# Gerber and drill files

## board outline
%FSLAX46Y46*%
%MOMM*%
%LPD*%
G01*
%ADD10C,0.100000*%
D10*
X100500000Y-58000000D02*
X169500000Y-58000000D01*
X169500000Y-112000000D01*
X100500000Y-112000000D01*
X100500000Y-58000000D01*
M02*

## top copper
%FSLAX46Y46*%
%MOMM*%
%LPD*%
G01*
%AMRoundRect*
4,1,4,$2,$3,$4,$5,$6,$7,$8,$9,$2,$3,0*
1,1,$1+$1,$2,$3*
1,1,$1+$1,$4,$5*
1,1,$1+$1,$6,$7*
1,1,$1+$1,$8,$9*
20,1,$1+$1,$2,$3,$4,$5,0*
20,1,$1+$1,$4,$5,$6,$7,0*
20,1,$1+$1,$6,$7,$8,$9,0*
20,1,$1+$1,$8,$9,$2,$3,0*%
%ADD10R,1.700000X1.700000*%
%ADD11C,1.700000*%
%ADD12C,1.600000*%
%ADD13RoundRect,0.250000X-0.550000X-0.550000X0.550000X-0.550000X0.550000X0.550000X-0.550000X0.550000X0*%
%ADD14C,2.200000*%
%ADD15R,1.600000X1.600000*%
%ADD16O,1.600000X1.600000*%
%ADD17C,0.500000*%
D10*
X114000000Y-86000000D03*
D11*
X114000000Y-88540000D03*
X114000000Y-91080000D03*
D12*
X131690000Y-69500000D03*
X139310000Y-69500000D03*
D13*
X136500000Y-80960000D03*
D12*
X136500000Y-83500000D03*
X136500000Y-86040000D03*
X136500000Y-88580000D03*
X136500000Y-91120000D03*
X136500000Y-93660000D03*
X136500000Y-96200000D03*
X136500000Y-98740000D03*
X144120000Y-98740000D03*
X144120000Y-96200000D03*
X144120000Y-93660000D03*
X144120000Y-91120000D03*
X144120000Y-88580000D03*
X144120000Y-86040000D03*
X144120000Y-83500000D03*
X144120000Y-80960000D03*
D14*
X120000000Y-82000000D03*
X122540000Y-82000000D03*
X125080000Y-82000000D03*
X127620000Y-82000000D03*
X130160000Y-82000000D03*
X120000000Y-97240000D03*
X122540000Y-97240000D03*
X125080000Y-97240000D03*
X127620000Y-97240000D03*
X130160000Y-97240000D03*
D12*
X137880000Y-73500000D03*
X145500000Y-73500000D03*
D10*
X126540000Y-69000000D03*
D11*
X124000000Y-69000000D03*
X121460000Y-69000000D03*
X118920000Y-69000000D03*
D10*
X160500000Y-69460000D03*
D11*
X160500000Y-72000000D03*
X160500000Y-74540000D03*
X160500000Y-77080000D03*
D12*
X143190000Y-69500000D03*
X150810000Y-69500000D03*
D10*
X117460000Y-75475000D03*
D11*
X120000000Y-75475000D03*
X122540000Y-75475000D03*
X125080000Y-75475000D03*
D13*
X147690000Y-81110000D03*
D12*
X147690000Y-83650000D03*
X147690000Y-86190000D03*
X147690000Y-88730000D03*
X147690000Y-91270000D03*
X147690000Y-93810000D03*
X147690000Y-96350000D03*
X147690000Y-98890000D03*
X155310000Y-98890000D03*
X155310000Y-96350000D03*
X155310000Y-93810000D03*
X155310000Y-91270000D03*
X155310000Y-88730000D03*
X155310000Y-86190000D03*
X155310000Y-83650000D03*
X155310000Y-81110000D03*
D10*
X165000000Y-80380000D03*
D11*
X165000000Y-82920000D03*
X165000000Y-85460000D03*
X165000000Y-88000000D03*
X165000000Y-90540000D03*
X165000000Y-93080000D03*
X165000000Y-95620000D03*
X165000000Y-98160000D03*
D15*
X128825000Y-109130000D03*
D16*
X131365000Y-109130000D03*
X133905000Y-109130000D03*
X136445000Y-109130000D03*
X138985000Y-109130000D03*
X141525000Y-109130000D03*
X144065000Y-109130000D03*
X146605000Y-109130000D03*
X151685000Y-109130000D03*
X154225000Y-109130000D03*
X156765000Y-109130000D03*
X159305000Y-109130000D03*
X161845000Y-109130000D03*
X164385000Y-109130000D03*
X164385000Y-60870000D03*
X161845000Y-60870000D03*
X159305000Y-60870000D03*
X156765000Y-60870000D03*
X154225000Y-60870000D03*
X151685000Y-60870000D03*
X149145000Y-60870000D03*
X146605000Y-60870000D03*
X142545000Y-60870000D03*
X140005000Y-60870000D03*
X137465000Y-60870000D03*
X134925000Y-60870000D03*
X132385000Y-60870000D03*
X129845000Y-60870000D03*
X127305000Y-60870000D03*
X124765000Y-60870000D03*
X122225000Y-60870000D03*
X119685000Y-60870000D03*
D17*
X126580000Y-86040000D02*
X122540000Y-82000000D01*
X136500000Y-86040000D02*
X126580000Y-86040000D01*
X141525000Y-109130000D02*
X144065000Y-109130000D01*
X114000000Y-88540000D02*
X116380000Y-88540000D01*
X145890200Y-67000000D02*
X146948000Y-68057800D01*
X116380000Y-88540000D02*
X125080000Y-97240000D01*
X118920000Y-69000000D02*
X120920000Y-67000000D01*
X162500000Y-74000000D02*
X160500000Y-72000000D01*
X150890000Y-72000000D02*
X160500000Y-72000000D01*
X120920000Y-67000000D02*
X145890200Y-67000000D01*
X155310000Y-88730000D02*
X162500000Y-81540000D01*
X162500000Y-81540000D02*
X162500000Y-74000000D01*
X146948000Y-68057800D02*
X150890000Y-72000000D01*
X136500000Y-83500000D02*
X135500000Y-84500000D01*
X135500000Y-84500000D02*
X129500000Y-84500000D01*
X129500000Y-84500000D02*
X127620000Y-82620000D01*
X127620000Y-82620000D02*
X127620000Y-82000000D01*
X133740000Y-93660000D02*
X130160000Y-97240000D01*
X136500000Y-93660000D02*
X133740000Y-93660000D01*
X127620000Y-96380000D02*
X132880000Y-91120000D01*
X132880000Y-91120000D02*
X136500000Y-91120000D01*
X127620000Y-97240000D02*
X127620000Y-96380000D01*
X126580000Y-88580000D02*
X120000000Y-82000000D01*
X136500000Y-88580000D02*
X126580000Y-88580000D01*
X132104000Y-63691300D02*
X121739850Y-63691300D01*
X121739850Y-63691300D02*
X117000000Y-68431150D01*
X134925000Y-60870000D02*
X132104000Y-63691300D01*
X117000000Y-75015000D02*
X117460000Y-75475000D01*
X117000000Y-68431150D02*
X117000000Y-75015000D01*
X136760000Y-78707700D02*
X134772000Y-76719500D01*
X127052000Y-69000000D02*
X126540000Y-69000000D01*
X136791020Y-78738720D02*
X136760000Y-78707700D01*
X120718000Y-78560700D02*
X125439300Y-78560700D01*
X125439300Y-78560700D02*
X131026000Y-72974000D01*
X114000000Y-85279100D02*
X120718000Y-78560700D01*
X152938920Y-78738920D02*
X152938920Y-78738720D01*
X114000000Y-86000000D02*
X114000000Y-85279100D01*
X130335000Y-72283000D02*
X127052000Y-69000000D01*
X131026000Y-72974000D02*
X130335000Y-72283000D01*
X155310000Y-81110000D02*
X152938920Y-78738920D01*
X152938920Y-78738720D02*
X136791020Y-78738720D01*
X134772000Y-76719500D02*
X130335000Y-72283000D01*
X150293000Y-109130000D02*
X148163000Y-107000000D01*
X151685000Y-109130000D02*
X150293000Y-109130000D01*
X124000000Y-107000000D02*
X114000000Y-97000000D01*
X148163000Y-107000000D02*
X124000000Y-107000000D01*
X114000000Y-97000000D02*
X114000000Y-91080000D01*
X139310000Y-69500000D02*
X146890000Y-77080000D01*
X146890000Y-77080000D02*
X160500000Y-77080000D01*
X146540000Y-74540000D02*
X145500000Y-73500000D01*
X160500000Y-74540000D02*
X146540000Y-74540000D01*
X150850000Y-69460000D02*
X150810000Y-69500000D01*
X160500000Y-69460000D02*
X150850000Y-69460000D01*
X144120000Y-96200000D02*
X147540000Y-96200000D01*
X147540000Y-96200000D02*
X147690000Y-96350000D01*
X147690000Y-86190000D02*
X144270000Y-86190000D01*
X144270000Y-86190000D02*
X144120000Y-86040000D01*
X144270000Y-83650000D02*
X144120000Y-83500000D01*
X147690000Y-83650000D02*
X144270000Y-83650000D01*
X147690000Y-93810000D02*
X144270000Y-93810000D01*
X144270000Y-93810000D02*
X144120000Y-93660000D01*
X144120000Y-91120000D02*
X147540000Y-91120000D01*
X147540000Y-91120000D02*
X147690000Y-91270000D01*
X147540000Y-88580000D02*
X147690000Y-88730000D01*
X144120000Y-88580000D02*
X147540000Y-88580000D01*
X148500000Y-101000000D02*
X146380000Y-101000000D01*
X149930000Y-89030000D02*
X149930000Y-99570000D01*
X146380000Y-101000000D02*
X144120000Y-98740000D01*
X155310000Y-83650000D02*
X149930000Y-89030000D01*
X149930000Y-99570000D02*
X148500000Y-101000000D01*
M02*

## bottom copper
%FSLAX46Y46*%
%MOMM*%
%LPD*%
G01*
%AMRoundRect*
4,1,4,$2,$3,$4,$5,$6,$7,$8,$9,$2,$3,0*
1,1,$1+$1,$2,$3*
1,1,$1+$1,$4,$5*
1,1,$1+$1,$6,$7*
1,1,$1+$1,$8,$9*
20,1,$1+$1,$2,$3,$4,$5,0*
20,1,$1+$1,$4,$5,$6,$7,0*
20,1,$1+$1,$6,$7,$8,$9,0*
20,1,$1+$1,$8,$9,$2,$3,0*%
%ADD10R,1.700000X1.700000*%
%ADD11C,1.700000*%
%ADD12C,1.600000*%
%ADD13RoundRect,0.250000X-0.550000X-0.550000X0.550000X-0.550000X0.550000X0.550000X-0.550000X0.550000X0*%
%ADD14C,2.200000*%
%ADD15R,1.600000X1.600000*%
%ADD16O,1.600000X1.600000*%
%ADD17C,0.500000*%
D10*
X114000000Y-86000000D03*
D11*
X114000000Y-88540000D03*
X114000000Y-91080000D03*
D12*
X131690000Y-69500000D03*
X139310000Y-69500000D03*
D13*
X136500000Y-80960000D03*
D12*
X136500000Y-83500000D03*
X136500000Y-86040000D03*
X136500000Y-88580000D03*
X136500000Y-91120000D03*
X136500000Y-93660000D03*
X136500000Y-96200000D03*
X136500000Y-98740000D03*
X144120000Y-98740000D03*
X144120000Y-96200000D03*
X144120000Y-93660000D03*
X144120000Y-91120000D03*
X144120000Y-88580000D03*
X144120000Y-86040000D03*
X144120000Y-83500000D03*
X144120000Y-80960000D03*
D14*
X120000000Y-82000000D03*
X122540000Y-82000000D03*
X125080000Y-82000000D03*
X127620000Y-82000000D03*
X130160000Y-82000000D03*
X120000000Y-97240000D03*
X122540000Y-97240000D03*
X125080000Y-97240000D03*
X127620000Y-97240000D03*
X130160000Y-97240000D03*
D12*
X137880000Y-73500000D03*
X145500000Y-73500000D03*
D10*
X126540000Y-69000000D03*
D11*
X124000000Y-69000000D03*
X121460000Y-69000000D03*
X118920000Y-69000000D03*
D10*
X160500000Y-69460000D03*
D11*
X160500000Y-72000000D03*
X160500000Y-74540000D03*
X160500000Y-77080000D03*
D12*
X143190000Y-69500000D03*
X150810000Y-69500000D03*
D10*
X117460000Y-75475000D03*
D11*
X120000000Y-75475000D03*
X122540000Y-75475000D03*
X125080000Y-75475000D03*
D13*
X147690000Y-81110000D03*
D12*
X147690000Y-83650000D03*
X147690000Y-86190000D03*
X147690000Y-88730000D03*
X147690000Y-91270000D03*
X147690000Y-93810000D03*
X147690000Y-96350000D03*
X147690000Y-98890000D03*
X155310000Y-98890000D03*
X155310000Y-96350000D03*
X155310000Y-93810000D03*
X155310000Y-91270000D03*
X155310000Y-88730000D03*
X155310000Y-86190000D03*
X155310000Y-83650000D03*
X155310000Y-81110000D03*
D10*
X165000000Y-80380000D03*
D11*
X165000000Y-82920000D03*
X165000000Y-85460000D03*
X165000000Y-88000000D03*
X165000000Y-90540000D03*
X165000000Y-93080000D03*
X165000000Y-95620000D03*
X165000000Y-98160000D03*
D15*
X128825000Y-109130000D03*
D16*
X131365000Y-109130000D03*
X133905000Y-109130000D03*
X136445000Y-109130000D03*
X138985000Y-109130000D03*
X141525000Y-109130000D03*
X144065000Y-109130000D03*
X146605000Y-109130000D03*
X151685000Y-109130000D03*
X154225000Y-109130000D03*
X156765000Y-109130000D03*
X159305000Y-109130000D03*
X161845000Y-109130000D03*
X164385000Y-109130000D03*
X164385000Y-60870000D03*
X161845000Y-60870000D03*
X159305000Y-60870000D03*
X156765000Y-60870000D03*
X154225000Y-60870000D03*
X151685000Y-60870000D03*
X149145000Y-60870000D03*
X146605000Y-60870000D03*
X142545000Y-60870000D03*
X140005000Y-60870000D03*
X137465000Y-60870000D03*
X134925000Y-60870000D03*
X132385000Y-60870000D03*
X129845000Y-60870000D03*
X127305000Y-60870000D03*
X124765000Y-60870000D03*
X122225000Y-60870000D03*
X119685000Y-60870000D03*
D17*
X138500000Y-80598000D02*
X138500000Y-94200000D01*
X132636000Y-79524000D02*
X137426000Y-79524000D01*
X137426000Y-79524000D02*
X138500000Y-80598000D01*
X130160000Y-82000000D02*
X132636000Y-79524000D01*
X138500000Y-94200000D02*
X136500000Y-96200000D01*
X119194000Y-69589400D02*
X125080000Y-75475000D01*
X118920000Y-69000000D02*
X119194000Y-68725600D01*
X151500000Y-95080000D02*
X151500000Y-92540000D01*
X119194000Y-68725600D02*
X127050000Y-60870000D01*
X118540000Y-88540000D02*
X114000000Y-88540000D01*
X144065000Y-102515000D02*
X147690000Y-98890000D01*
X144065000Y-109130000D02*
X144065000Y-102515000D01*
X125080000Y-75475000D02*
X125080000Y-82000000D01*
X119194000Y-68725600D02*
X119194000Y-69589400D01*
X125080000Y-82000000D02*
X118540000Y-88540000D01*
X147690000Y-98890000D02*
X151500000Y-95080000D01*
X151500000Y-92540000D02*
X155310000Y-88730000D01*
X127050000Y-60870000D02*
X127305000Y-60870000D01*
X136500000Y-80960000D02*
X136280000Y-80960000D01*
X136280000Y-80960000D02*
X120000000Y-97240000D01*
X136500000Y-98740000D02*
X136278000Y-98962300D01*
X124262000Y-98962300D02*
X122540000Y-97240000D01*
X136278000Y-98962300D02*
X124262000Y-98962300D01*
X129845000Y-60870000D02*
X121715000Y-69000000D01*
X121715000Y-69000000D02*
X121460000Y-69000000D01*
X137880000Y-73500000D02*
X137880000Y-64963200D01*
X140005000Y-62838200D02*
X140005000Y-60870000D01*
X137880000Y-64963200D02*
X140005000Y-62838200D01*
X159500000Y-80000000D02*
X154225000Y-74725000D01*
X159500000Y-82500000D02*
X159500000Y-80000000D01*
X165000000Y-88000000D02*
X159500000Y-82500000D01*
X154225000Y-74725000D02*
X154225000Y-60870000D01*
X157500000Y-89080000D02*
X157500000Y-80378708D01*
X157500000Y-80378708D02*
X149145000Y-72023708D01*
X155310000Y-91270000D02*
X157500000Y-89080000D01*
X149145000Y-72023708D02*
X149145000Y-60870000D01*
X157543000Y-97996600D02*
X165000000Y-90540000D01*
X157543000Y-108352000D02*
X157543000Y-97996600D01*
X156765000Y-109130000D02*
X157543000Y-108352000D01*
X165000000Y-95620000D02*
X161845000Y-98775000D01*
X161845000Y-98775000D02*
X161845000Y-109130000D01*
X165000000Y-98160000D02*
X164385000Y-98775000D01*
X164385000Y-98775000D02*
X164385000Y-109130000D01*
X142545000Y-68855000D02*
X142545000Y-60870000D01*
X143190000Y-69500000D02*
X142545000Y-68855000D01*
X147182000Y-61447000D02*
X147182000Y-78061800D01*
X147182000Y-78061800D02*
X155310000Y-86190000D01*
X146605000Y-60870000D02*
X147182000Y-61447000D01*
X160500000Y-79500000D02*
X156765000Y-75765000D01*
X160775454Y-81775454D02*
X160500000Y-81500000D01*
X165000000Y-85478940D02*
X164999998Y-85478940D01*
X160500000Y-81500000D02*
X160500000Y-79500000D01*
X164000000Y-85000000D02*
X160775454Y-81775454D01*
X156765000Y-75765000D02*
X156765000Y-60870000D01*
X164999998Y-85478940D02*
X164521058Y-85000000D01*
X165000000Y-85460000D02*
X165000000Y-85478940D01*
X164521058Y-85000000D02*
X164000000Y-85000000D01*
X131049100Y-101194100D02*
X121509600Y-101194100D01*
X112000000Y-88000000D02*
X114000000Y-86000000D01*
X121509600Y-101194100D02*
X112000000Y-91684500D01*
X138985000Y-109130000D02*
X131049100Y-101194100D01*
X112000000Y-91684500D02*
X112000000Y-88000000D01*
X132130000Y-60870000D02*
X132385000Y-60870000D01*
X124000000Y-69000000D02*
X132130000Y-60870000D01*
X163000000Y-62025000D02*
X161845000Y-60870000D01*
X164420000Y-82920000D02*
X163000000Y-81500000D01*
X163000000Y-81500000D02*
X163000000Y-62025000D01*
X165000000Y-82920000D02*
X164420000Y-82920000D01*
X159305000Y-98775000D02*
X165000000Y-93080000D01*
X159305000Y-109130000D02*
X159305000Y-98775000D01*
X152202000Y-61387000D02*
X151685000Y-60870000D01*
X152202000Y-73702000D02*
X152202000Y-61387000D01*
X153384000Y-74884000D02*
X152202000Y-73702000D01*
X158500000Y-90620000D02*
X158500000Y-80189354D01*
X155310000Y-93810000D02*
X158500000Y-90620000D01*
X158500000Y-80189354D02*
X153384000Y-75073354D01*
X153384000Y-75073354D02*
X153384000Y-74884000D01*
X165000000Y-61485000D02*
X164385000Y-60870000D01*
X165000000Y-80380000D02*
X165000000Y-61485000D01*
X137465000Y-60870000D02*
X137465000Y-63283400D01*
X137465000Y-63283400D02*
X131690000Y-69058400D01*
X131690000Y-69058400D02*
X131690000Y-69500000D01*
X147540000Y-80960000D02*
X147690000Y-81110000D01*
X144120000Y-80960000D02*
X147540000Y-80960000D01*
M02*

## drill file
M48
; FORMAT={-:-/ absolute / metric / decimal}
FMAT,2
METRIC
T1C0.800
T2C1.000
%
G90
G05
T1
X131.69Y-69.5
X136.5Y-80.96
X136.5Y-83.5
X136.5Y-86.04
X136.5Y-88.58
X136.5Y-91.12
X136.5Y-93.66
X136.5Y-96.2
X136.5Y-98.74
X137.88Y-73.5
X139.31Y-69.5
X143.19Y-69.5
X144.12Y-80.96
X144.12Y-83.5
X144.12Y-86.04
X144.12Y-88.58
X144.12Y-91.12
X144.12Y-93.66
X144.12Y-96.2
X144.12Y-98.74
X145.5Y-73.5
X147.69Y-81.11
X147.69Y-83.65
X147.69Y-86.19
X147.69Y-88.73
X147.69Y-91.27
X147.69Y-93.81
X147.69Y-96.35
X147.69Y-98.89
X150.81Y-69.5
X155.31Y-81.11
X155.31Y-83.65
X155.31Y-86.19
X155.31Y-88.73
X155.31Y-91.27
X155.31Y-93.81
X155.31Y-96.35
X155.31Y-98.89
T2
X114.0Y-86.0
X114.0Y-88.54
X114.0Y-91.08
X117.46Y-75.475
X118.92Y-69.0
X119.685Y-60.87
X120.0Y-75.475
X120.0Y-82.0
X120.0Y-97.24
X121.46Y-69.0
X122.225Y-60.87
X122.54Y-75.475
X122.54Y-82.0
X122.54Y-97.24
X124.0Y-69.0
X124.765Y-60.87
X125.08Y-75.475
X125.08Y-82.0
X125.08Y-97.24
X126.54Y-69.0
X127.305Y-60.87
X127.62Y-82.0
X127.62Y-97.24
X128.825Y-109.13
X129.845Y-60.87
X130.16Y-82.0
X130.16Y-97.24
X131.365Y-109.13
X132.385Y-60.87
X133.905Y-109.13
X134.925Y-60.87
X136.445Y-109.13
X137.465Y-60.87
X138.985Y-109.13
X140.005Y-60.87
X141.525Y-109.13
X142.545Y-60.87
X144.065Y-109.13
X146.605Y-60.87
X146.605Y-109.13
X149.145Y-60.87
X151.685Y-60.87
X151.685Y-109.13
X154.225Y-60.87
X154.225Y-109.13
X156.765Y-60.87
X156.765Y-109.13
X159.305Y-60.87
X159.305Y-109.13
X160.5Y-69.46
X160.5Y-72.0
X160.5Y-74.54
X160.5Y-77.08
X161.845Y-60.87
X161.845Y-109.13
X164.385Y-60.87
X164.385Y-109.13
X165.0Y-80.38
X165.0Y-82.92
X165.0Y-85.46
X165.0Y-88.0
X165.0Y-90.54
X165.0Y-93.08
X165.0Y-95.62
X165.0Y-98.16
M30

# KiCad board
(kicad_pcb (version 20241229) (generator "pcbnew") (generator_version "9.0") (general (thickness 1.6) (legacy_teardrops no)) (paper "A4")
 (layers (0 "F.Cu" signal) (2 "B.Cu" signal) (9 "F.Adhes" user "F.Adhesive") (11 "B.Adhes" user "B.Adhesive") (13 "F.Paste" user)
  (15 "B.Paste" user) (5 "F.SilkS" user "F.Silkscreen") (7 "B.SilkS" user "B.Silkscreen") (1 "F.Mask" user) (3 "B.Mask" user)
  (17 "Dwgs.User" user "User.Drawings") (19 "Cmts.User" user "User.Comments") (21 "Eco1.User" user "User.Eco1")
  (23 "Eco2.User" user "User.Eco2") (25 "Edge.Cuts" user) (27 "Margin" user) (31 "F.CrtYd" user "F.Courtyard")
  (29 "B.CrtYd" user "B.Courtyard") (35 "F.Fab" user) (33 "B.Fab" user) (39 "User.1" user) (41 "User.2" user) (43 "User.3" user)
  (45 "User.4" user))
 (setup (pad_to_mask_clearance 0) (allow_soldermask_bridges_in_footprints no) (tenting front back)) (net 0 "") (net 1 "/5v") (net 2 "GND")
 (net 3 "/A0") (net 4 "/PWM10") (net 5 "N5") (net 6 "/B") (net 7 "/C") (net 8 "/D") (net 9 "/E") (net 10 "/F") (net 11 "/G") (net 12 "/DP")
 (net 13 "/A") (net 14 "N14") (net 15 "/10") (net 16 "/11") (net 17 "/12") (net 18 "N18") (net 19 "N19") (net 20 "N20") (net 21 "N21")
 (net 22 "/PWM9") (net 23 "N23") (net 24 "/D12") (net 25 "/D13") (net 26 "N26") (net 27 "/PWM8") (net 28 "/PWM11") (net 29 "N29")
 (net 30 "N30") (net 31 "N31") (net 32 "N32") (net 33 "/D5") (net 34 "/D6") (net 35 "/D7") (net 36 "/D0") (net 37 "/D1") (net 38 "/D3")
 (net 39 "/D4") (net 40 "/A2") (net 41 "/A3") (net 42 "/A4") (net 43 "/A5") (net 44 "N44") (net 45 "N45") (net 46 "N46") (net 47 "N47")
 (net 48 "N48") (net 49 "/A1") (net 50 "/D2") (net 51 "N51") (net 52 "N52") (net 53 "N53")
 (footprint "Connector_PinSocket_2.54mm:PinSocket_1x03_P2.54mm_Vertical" (layer "F.Cu") (at 114 86)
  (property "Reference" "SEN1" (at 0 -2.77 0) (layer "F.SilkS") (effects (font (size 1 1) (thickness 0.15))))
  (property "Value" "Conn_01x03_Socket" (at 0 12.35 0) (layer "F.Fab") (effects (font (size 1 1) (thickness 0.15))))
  (pad "1" thru_hole rect (at 0 0) (size 1.7 1.7) (drill 1) (layers "*.Cu" "*.Mask") (remove_unused_layers no) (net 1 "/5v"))
  (pad "2" thru_hole circle (at 0 2.54) (size 1.7 1.7) (drill 1) (layers "*.Cu" "*.Mask") (remove_unused_layers no) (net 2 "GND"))
  (pad "3" thru_hole circle (at 0 5.08) (size 1.7 1.7) (drill 1) (layers "*.Cu" "*.Mask") (remove_unused_layers no) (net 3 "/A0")))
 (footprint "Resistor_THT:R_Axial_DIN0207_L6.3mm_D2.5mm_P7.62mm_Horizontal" (layer "F.Cu") (at 131.69 69.5)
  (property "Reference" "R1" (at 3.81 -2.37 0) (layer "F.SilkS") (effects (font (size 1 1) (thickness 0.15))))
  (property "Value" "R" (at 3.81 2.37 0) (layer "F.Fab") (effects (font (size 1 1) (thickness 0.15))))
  (pad "1" thru_hole circle (at 0 0) (size 1.6 1.6) (drill 0.8) (layers "*.Cu" "*.Mask") (remove_unused_layers no) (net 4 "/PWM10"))
  (pad "2" thru_hole circle (at 7.62 0) (size 1.6 1.6) (drill 0.8) (layers "*.Cu" "*.Mask") (remove_unused_layers no) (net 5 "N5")))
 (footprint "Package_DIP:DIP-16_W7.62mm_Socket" (layer "F.Cu") (at 136.5 80.96)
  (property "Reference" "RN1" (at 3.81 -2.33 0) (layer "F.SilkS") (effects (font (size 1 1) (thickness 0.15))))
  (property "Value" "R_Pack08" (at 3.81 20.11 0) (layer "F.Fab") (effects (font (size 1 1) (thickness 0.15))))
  (pad "1" thru_hole roundrect (at 0 0) (size 1.6 1.6) (drill 0.8) (layers "*.Cu" "*.Mask") (remove_unused_layers no)
   (roundrect_rratio 0.15625) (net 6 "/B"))
  (pad "2" thru_hole circle (at 0 2.54) (size 1.6 1.6) (drill 0.8) (layers "*.Cu" "*.Mask") (remove_unused_layers no) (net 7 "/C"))
  (pad "3" thru_hole circle (at 0 5.08) (size 1.6 1.6) (drill 0.8) (layers "*.Cu" "*.Mask") (remove_unused_layers no) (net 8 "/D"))
  (pad "4" thru_hole circle (at 0 7.62) (size 1.6 1.6) (drill 0.8) (layers "*.Cu" "*.Mask") (remove_unused_layers no) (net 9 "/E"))
  (pad "5" thru_hole circle (at 0 10.16) (size 1.6 1.6) (drill 0.8) (layers "*.Cu" "*.Mask") (remove_unused_layers no) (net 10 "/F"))
  (pad "6" thru_hole circle (at 0 12.7) (size 1.6 1.6) (drill 0.8) (layers "*.Cu" "*.Mask") (remove_unused_layers no) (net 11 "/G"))
  (pad "7" thru_hole circle (at 0 15.24) (size 1.6 1.6) (drill 0.8) (layers "*.Cu" "*.Mask") (remove_unused_layers no) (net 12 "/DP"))
  (pad "8" thru_hole circle (at 0 17.78) (size 1.6 1.6) (drill 0.8) (layers "*.Cu" "*.Mask") (remove_unused_layers no) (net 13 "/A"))
  (pad "9" thru_hole circle (at 7.62 17.78) (size 1.6 1.6) (drill 0.8) (layers "*.Cu" "*.Mask") (remove_unused_layers no) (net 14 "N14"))
  (pad "10" thru_hole circle (at 7.62 15.24) (size 1.6 1.6) (drill 0.8) (layers "*.Cu" "*.Mask") (remove_unused_layers no) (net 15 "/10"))
  (pad "11" thru_hole circle (at 7.62 12.7) (size 1.6 1.6) (drill 0.8) (layers "*.Cu" "*.Mask") (remove_unused_layers no) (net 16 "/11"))
  (pad "12" thru_hole circle (at 7.62 10.16) (size 1.6 1.6) (drill 0.8) (layers "*.Cu" "*.Mask") (remove_unused_layers no) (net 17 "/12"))
  (pad "13" thru_hole circle (at 7.62 7.62) (size 1.6 1.6) (drill 0.8) (layers "*.Cu" "*.Mask") (remove_unused_layers no) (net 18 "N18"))
  (pad "14" thru_hole circle (at 7.62 5.08) (size 1.6 1.6) (drill 0.8) (layers "*.Cu" "*.Mask") (remove_unused_layers no) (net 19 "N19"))
  (pad "15" thru_hole circle (at 7.62 2.54) (size 1.6 1.6) (drill 0.8) (layers "*.Cu" "*.Mask") (remove_unused_layers no) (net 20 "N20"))
  (pad "16" thru_hole circle (at 7.62 0) (size 1.6 1.6) (drill 0.8) (layers "*.Cu" "*.Mask") (remove_unused_layers no) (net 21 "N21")))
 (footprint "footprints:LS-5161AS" (layer "F.Cu") (at 120 82)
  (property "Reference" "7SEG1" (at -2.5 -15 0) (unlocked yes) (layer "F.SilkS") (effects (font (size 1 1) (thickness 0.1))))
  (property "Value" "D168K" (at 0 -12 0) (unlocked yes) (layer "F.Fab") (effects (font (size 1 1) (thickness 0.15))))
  (pad "1" thru_hole circle (at 0 0) (size 2.2 2.2) (drill 1) (layers "*.Cu" "*.Mask") (remove_unused_layers no) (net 9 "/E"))
  (pad "2" thru_hole circle (at 2.54 0) (size 2.2 2.2) (drill 1) (layers "*.Cu" "*.Mask") (remove_unused_layers no) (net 8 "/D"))
  (pad "3" thru_hole circle (at 5.08 0) (size 2.2 2.2) (drill 1) (layers "*.Cu" "*.Mask") (remove_unused_layers no) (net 2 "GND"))
  (pad "4" thru_hole circle (at 7.62 0) (size 2.2 2.2) (drill 1) (layers "*.Cu" "*.Mask") (remove_unused_layers no) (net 7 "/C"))
  (pad "5" thru_hole circle (at 10.16 0) (size 2.2 2.2) (drill 1) (layers "*.Cu" "*.Mask") (remove_unused_layers no) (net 12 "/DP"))
  (pad "6" thru_hole circle (at 0 15.24) (size 2.2 2.2) (drill 1) (layers "*.Cu" "*.Mask") (remove_unused_layers no) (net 6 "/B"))
  (pad "7" thru_hole circle (at 2.54 15.24) (size 2.2 2.2) (drill 1) (layers "*.Cu" "*.Mask") (remove_unused_layers no) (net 13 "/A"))
  (pad "8" thru_hole circle (at 5.08 15.24) (size 2.2 2.2) (drill 1) (layers "*.Cu" "*.Mask") (remove_unused_layers no) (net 2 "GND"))
  (pad "9" thru_hole circle (at 7.62 15.24) (size 2.2 2.2) (drill 1) (layers "*.Cu" "*.Mask") (remove_unused_layers no) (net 10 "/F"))
  (pad "10" thru_hole circle (at 10.16 15.24) (size 2.2 2.2) (drill 1) (layers "*.Cu" "*.Mask") (remove_unused_layers no) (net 11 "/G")))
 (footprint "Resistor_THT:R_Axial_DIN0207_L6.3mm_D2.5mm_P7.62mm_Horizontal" (layer "F.Cu") (at 137.88 73.5)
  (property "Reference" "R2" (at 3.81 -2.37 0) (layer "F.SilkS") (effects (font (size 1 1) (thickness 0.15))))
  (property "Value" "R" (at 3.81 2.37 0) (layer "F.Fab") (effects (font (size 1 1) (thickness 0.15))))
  (pad "1" thru_hole circle (at 0 0) (size 1.6 1.6) (drill 0.8) (layers "*.Cu" "*.Mask") (remove_unused_layers no) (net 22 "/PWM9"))
  (pad "2" thru_hole circle (at 7.62 0) (size 1.6 1.6) (drill 0.8) (layers "*.Cu" "*.Mask") (remove_unused_layers no) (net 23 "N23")))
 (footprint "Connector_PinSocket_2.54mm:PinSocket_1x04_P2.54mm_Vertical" (layer "F.Cu") (at 126.54 69 -90)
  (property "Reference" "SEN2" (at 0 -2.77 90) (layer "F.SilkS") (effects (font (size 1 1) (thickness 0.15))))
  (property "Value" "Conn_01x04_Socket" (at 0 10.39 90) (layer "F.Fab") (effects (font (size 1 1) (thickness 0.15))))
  (pad "1" thru_hole rect (at 0 0 270) (size 1.7 1.7) (drill 1) (layers "*.Cu" "*.Mask") (remove_unused_layers no) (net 1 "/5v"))
  (pad "2" thru_hole circle (at 0 2.54 270) (size 1.7 1.7) (drill 1) (layers "*.Cu" "*.Mask") (remove_unused_layers no) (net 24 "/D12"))
  (pad "3" thru_hole circle (at 0 5.08 270) (size 1.7 1.7) (drill 1) (layers "*.Cu" "*.Mask") (remove_unused_layers no) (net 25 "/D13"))
  (pad "4" thru_hole circle (at 0 7.62 270) (size 1.7 1.7) (drill 1) (layers "*.Cu" "*.Mask") (remove_unused_layers no) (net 2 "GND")))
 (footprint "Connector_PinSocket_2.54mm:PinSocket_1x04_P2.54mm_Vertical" (layer "F.Cu") (at 160.5 69.46)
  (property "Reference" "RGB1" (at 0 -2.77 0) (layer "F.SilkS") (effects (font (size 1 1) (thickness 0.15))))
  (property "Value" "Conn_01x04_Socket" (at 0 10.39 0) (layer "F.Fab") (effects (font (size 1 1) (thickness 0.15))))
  (pad "1" thru_hole rect (at 0 0) (size 1.7 1.7) (drill 1) (layers "*.Cu" "*.Mask") (remove_unused_layers no) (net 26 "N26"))
  (pad "2" thru_hole circle (at 0 2.54) (size 1.7 1.7) (drill 1) (layers "*.Cu" "*.Mask") (remove_unused_layers no) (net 2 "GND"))
  (pad "3" thru_hole circle (at 0 5.08) (size 1.7 1.7) (drill 1) (layers "*.Cu" "*.Mask") (remove_unused_layers no) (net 23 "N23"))
  (pad "4" thru_hole circle (at 0 7.62) (size 1.7 1.7) (drill 1) (layers "*.Cu" "*.Mask") (remove_unused_layers no) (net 5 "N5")))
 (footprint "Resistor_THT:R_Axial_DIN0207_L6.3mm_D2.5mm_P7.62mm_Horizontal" (layer "F.Cu") (at 143.19 69.5)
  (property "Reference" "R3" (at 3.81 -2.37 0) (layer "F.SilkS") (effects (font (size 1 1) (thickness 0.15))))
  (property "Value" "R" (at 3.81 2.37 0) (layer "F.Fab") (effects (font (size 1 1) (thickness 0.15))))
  (pad "1" thru_hole circle (at 0 0) (size 1.6 1.6) (drill 0.8) (layers "*.Cu" "*.Mask") (remove_unused_layers no) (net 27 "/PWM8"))
  (pad "2" thru_hole circle (at 7.62 0) (size 1.6 1.6) (drill 0.8) (layers "*.Cu" "*.Mask") (remove_unused_layers no) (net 26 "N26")))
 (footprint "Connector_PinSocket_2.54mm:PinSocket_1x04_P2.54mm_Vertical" (layer "F.Cu") (at 117.46 75.475 90)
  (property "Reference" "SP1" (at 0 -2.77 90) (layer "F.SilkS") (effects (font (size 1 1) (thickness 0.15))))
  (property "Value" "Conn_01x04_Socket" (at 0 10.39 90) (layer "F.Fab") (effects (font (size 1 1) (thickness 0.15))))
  (pad "1" thru_hole rect (at 0 0 90) (size 1.7 1.7) (drill 1) (layers "*.Cu" "*.Mask") (remove_unused_layers no) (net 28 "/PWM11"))
  (pad "2" thru_hole circle (at 0 2.54 90) (size 1.7 1.7) (drill 1) (layers "*.Cu" "*.Mask") (remove_unused_layers no) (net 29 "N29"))
  (pad "3" thru_hole circle (at 0 5.08 90) (size 1.7 1.7) (drill 1) (layers "*.Cu" "*.Mask") (remove_unused_layers no) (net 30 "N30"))
  (pad "4" thru_hole circle (at 0 7.62 90) (size 1.7 1.7) (drill 1) (layers "*.Cu" "*.Mask") (remove_unused_layers no) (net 2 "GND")))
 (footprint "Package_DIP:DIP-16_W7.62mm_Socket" (layer "F.Cu") (at 147.69 81.11)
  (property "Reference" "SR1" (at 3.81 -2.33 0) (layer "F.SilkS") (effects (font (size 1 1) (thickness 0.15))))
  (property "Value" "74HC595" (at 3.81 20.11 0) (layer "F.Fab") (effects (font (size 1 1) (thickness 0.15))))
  (pad "1" thru_hole roundrect (at 0 0) (size 1.6 1.6) (drill 0.8) (layers "*.Cu" "*.Mask") (remove_unused_layers no)
   (roundrect_rratio 0.15625) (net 21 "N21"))
  (pad "2" thru_hole circle (at 0 2.54) (size 1.6 1.6) (drill 0.8) (layers "*.Cu" "*.Mask") (remove_unused_layers no) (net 20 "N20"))
  (pad "3" thru_hole circle (at 0 5.08) (size 1.6 1.6) (drill 0.8) (layers "*.Cu" "*.Mask") (remove_unused_layers no) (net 19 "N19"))
  (pad "4" thru_hole circle (at 0 7.62) (size 1.6 1.6) (drill 0.8) (layers "*.Cu" "*.Mask") (remove_unused_layers no) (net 18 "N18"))
  (pad "5" thru_hole circle (at 0 10.16) (size 1.6 1.6) (drill 0.8) (layers "*.Cu" "*.Mask") (remove_unused_layers no) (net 17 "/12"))
  (pad "6" thru_hole circle (at 0 12.7) (size 1.6 1.6) (drill 0.8) (layers "*.Cu" "*.Mask") (remove_unused_layers no) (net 16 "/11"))
  (pad "7" thru_hole circle (at 0 15.24) (size 1.6 1.6) (drill 0.8) (layers "*.Cu" "*.Mask") (remove_unused_layers no) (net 15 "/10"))
  (pad "8" thru_hole circle (at 0 17.78) (size 1.6 1.6) (drill 0.8) (layers "*.Cu" "*.Mask") (remove_unused_layers no) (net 2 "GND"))
  (pad "9" thru_hole circle (at 7.62 17.78) (size 1.6 1.6) (drill 0.8) (layers "*.Cu" "*.Mask") (remove_unused_layers no) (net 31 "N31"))
  (pad "10" thru_hole circle (at 7.62 15.24) (size 1.6 1.6) (drill 0.8) (layers "*.Cu" "*.Mask") (remove_unused_layers no) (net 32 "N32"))
  (pad "11" thru_hole circle (at 7.62 12.7) (size 1.6 1.6) (drill 0.8) (layers "*.Cu" "*.Mask") (remove_unused_layers no) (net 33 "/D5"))
  (pad "12" thru_hole circle (at 7.62 10.16) (size 1.6 1.6) (drill 0.8) (layers "*.Cu" "*.Mask") (remove_unused_layers no) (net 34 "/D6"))
  (pad "13" thru_hole circle (at 7.62 7.62) (size 1.6 1.6) (drill 0.8) (layers "*.Cu" "*.Mask") (remove_unused_layers no) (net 2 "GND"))
  (pad "14" thru_hole circle (at 7.62 5.08) (size 1.6 1.6) (drill 0.8) (layers "*.Cu" "*.Mask") (remove_unused_layers no) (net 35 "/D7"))
  (pad "15" thru_hole circle (at 7.62 2.54) (size 1.6 1.6) (drill 0.8) (layers "*.Cu" "*.Mask") (remove_unused_layers no) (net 14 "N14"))
  (pad "16" thru_hole circle (at 7.62 0) (size 1.6 1.6) (drill 0.8) (layers "*.Cu" "*.Mask") (remove_unused_layers no) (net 1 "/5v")))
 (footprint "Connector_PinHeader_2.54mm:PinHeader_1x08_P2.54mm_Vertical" (layer "F.Cu") (at 165 80.38)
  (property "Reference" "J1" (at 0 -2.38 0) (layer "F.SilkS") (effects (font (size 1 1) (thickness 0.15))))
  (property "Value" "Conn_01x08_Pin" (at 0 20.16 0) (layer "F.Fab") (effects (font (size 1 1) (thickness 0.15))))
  (pad "1" thru_hole rect (at 0 0) (size 1.7 1.7) (drill 1) (layers "*.Cu" "*.Mask") (remove_unused_layers no) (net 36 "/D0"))
  (pad "2" thru_hole circle (at 0 2.54) (size 1.7 1.7) (drill 1) (layers "*.Cu" "*.Mask") (remove_unused_layers no) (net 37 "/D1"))
  (pad "3" thru_hole circle (at 0 5.08) (size 1.7 1.7) (drill 1) (layers "*.Cu" "*.Mask") (remove_unused_layers no) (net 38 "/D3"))
  (pad "4" thru_hole circle (at 0 7.62) (size 1.7 1.7) (drill 1) (layers "*.Cu" "*.Mask") (remove_unused_layers no) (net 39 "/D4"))
  (pad "5" thru_hole circle (at 0 10.16) (size 1.7 1.7) (drill 1) (layers "*.Cu" "*.Mask") (remove_unused_layers no) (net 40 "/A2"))
  (pad "6" thru_hole circle (at 0 12.7) (size 1.7 1.7) (drill 1) (layers "*.Cu" "*.Mask") (remove_unused_layers no) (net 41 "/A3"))
  (pad "7" thru_hole circle (at 0 15.24) (size 1.7 1.7) (drill 1) (layers "*.Cu" "*.Mask") (remove_unused_layers no) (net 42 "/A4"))
  (pad "8" thru_hole circle (at 0 17.78) (size 1.7 1.7) (drill 1) (layers "*.Cu" "*.Mask") (remove_unused_layers no) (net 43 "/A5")))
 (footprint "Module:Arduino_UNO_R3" (layer "B.Cu") (at 128.825 109.13)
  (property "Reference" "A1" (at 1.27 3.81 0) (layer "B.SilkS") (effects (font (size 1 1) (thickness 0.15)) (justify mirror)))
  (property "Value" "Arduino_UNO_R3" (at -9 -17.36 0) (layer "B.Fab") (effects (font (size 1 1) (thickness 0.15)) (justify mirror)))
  (pad "1" thru_hole rect (at 0 0 270) (size 1.6 1.6) (drill 1) (layers "*.Cu" "*.Mask") (remove_unused_layers no) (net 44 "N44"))
  (pad "2" thru_hole oval (at 2.54 0 270) (size 1.6 1.6) (drill 1) (layers "*.Cu" "*.Mask") (remove_unused_layers no) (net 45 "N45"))
  (pad "3" thru_hole oval (at 5.08 0 270) (size 1.6 1.6) (drill 1) (layers "*.Cu" "*.Mask") (remove_unused_layers no) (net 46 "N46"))
  (pad "4" thru_hole oval (at 7.62 0 270) (size 1.6 1.6) (drill 1) (layers "*.Cu" "*.Mask") (remove_unused_layers no) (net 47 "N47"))
  (pad "5" thru_hole oval (at 10.16 0 270) (size 1.6 1.6) (drill 1) (layers "*.Cu" "*.Mask") (remove_unused_layers no) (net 1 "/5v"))
  (pad "6" thru_hole oval (at 12.7 0 270) (size 1.6 1.6) (drill 1) (layers "*.Cu" "*.Mask") (remove_unused_layers no) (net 2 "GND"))
  (pad "7" thru_hole oval (at 15.24 0 270) (size 1.6 1.6) (drill 1) (layers "*.Cu" "*.Mask") (remove_unused_layers no) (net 2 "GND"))
  (pad "8" thru_hole oval (at 17.78 0 270) (size 1.6 1.6) (drill 1) (layers "*.Cu" "*.Mask") (remove_unused_layers no) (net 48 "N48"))
  (pad "9" thru_hole oval (at 22.86 0 270) (size 1.6 1.6) (drill 1) (layers "*.Cu" "*.Mask") (remove_unused_layers no) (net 3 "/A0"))
  (pad "10" thru_hole oval (at 25.4 0 270) (size 1.6 1.6) (drill 1) (layers "*.Cu" "*.Mask") (remove_unused_layers no) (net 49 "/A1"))
  (pad "11" thru_hole oval (at 27.94 0 270) (size 1.6 1.6) (drill 1) (layers "*.Cu" "*.Mask") (remove_unused_layers no) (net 40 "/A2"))
  (pad "12" thru_hole oval (at 30.48 0 270) (size 1.6 1.6) (drill 1) (layers "*.Cu" "*.Mask") (remove_unused_layers no) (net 41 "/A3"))
  (pad "13" thru_hole oval (at 33.02 0 270) (size 1.6 1.6) (drill 1) (layers "*.Cu" "*.Mask") (remove_unused_layers no) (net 42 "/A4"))
  (pad "14" thru_hole oval (at 35.56 0 270) (size 1.6 1.6) (drill 1) (layers "*.Cu" "*.Mask") (remove_unused_layers no) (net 43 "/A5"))
  (pad "15" thru_hole oval (at 35.56 -48.26 270) (size 1.6 1.6) (drill 1) (layers "*.Cu" "*.Mask") (remove_unused_layers no) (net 36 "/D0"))
  (pad "16" thru_hole oval (at 33.02 -48.26 270) (size 1.6 1.6) (drill 1) (layers "*.Cu" "*.Mask") (remove_unused_layers no) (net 37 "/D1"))
  (pad "17" thru_hole oval (at 30.48 -48.26 270) (size 1.6 1.6) (drill 1) (layers "*.Cu" "*.Mask") (remove_unused_layers no) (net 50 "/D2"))
  (pad "18" thru_hole oval (at 27.94 -48.26 270) (size 1.6 1.6) (drill 1) (layers "*.Cu" "*.Mask") (remove_unused_layers no) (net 38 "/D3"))
  (pad "19" thru_hole oval (at 25.4 -48.26 270) (size 1.6 1.6) (drill 1) (layers "*.Cu" "*.Mask") (remove_unused_layers no) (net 39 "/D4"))
  (pad "20" thru_hole oval (at 22.86 -48.26 270) (size 1.6 1.6) (drill 1) (layers "*.Cu" "*.Mask") (remove_unused_layers no) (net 33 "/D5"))
  (pad "21" thru_hole oval (at 20.32 -48.26 270) (size 1.6 1.6) (drill 1) (layers "*.Cu" "*.Mask") (remove_unused_layers no) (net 34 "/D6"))
  (pad "22" thru_hole oval (at 17.78 -48.26 270) (size 1.6 1.6) (drill 1) (layers "*.Cu" "*.Mask") (remove_unused_layers no) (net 35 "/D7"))
  (pad "23" thru_hole oval (at 13.72 -48.26 270) (size 1.6 1.6) (drill 1) (layers "*.Cu" "*.Mask") (remove_unused_layers no)
   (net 27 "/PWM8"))
  (pad "24" thru_hole oval (at 11.18 -48.26 270) (size 1.6 1.6) (drill 1) (layers "*.Cu" "*.Mask") (remove_unused_layers no)
   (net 22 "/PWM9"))
  (pad "25" thru_hole oval (at 8.64 -48.26 270) (size 1.6 1.6) (drill 1) (layers "*.Cu" "*.Mask") (remove_unused_layers no) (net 4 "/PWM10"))
  (pad "26" thru_hole oval (at 6.1 -48.26 270) (size 1.6 1.6) (drill 1) (layers "*.Cu" "*.Mask") (remove_unused_layers no) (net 28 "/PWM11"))
  (pad "27" thru_hole oval (at 3.56 -48.26 270) (size 1.6 1.6) (drill 1) (layers "*.Cu" "*.Mask") (remove_unused_layers no) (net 24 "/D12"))
  (pad "28" thru_hole oval (at 1.02 -48.26 270) (size 1.6 1.6) (drill 1) (layers "*.Cu" "*.Mask") (remove_unused_layers no) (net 25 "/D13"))
  (pad "29" thru_hole oval (at -1.52 -48.26 270) (size 1.6 1.6) (drill 1) (layers "*.Cu" "*.Mask") (remove_unused_layers no) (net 2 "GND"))
  (pad "30" thru_hole oval (at -4.06 -48.26 270) (size 1.6 1.6) (drill 1) (layers "*.Cu" "*.Mask") (remove_unused_layers no) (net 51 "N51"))
  (pad "31" thru_hole oval (at -6.6 -48.26 270) (size 1.6 1.6) (drill 1) (layers "*.Cu" "*.Mask") (remove_unused_layers no) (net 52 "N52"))
  (pad "32" thru_hole oval (at -9.14 -48.26 270) (size 1.6 1.6) (drill 1) (layers "*.Cu" "*.Mask") (remove_unused_layers no) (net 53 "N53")))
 (gr_rect (start 100.5 58) (end 169.5 112) (stroke (width 0.1) (type default)) (fill no) (layer "Edge.Cuts"))
 (segment (start 138.5 80.598) (end 138.5 94.2) (width 0.5) (layer "B.Cu") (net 12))
 (segment (start 132.636 79.524) (end 137.426 79.524) (width 0.5) (layer "B.Cu") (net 12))
 (segment (start 137.426 79.524) (end 138.5 80.598) (width 0.5) (layer "B.Cu") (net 12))
 (segment (start 130.16 82) (end 132.636 79.524) (width 0.5) (layer "B.Cu") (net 12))
 (segment (start 138.5 94.2) (end 136.5 96.2) (width 0.5) (layer "B.Cu") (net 12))
 (segment (start 126.58 86.04) (end 122.54 82) (width 0.5) (layer "F.Cu") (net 8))
 (segment (start 136.5 86.04) (end 126.58 86.04) (width 0.5) (layer "F.Cu") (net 8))
 (segment (start 141.525 109.13) (end 144.065 109.13) (width 0.5) (layer "F.Cu") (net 2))
 (segment (start 114 88.54) (end 116.38 88.54) (width 0.5) (layer "F.Cu") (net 2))
 (segment (start 145.8902 67) (end 146.948 68.0578) (width 0.5) (layer "F.Cu") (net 2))
 (segment (start 116.38 88.54) (end 125.08 97.24) (width 0.5) (layer "F.Cu") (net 2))
 (segment (start 118.92 69) (end 120.92 67) (width 0.5) (layer "F.Cu") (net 2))
 (segment (start 162.5 74) (end 160.5 72) (width 0.5) (layer "F.Cu") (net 2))
 (segment (start 150.89 72) (end 160.5 72) (width 0.5) (layer "F.Cu") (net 2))
 (segment (start 120.92 67) (end 145.8902 67) (width 0.5) (layer "F.Cu") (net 2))
 (segment (start 155.31 88.73) (end 162.5 81.54) (width 0.5) (layer "F.Cu") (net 2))
 (segment (start 162.5 81.54) (end 162.5 74) (width 0.5) (layer "F.Cu") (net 2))
 (segment (start 146.948 68.0578) (end 150.89 72) (width 0.5) (layer "F.Cu") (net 2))
 (segment (start 119.194 69.5894) (end 125.08 75.475) (width 0.5) (layer "B.Cu") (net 2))
 (segment (start 118.92 69) (end 119.194 68.7256) (width 0.5) (layer "B.Cu") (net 2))
 (segment (start 151.5 95.08) (end 151.5 92.54) (width 0.5) (layer "B.Cu") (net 2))
 (segment (start 119.194 68.7256) (end 127.05 60.87) (width 0.5) (layer "B.Cu") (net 2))
 (segment (start 118.54 88.54) (end 114 88.54) (width 0.5) (layer "B.Cu") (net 2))
 (segment (start 144.065 102.515) (end 147.69 98.89) (width 0.5) (layer "B.Cu") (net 2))
 (segment (start 144.065 109.13) (end 144.065 102.515) (width 0.5) (layer "B.Cu") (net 2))
 (segment (start 125.08 75.475) (end 125.08 82) (width 0.5) (layer "B.Cu") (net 2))
 (segment (start 119.194 68.7256) (end 119.194 69.5894) (width 0.5) (layer "B.Cu") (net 2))
 (segment (start 125.08 82) (end 118.54 88.54) (width 0.5) (layer "B.Cu") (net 2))
 (segment (start 147.69 98.89) (end 151.5 95.08) (width 0.5) (layer "B.Cu") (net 2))
 (segment (start 151.5 92.54) (end 155.31 88.73) (width 0.5) (layer "B.Cu") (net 2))
 (segment (start 127.05 60.87) (end 127.305 60.87) (width 0.5) (layer "B.Cu") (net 2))
 (segment (start 136.5 83.5) (end 135.5 84.5) (width 0.5) (layer "F.Cu") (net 7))
 (segment (start 135.5 84.5) (end 129.5 84.5) (width 0.5) (layer "F.Cu") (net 7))
 (segment (start 129.5 84.5) (end 127.62 82.62) (width 0.5) (layer "F.Cu") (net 7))
 (segment (start 127.62 82.62) (end 127.62 82) (width 0.5) (layer "F.Cu") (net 7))
 (segment (start 136.5 80.96) (end 136.28 80.96) (width 0.5) (layer "B.Cu") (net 6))
 (segment (start 136.28 80.96) (end 120 97.24) (width 0.5) (layer "B.Cu") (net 6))
 (segment (start 136.5 98.74) (end 136.278 98.9623) (width 0.5) (layer "B.Cu") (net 13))
 (segment (start 124.262 98.9623) (end 122.54 97.24) (width 0.5) (layer "B.Cu") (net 13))
 (segment (start 136.278 98.9623) (end 124.262 98.9623) (width 0.5) (layer "B.Cu") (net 13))
 (segment (start 133.74 93.66) (end 130.16 97.24) (width 0.5) (layer "F.Cu") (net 11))
 (segment (start 136.5 93.66) (end 133.74 93.66) (width 0.5) (layer "F.Cu") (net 11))
 (segment (start 127.62 96.38) (end 132.88 91.12) (width 0.5) (layer "F.Cu") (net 10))
 (segment (start 132.88 91.12) (end 136.5 91.12) (width 0.5) (layer "F.Cu") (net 10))
 (segment (start 127.62 97.24) (end 127.62 96.38) (width 0.5) (layer "F.Cu") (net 10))
 (segment (start 126.58 88.58) (end 120 82) (width 0.5) (layer "F.Cu") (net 9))
 (segment (start 136.5 88.58) (end 126.58 88.58) (width 0.5) (layer "F.Cu") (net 9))
 (segment (start 129.845 60.87) (end 121.715 69) (width 0.5) (layer "B.Cu") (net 25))
 (segment (start 121.715 69) (end 121.46 69) (width 0.5) (layer "B.Cu") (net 25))
 (segment (start 137.88 73.5) (end 137.88 64.9632) (width 0.5) (layer "B.Cu") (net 22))
 (segment (start 140.005 62.8382) (end 140.005 60.87) (width 0.5) (layer "B.Cu") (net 22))
 (segment (start 137.88 64.9632) (end 140.005 62.8382) (width 0.5) (layer "B.Cu") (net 22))
 (segment (start 159.5 80) (end 154.225 74.725) (width 0.5) (layer "B.Cu") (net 39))
 (segment (start 159.5 82.5) (end 159.5 80) (width 0.5) (layer "B.Cu") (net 39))
 (segment (start 165 88) (end 159.5 82.5) (width 0.5) (layer "B.Cu") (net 39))
 (segment (start 154.225 74.725) (end 154.225 60.87) (width 0.5) (layer "B.Cu") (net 39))
 (segment (start 157.5 89.08) (end 157.5 80.378708) (width 0.5) (layer "B.Cu") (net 34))
 (segment (start 157.5 80.378708) (end 149.145 72.023708) (width 0.5) (layer "B.Cu") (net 34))
 (segment (start 155.31 91.27) (end 157.5 89.08) (width 0.5) (layer "B.Cu") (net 34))
 (segment (start 149.145 72.023708) (end 149.145 60.87) (width 0.5) (layer "B.Cu") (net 34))
 (segment (start 157.543 97.9966) (end 165 90.54) (width 0.5) (layer "B.Cu") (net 40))
 (segment (start 157.543 108.352) (end 157.543 97.9966) (width 0.5) (layer "B.Cu") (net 40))
 (segment (start 156.765 109.13) (end 157.543 108.352) (width 0.5) (layer "B.Cu") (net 40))
 (segment (start 165 95.62) (end 161.845 98.775) (width 0.5) (layer "B.Cu") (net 42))
 (segment (start 161.845 98.775) (end 161.845 109.13) (width 0.5) (layer "B.Cu") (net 42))
 (segment (start 165 98.16) (end 164.385 98.775) (width 0.5) (layer "B.Cu") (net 43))
 (segment (start 164.385 98.775) (end 164.385 109.13) (width 0.5) (layer "B.Cu") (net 43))
 (segment (start 132.104 63.6913) (end 121.73985 63.6913) (width 0.5) (layer "F.Cu") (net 28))
 (segment (start 121.73985 63.6913) (end 117 68.43115) (width 0.5) (layer "F.Cu") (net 28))
 (segment (start 134.925 60.87) (end 132.104 63.6913) (width 0.5) (layer "F.Cu") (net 28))
 (segment (start 117 75.015) (end 117.46 75.475) (width 0.5) (layer "F.Cu") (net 28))
 (segment (start 117 68.43115) (end 117 75.015) (width 0.5) (layer "F.Cu") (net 28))
 (segment (start 142.545 68.855) (end 142.545 60.87) (width 0.5) (layer "B.Cu") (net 27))
 (segment (start 143.19 69.5) (end 142.545 68.855) (width 0.5) (layer "B.Cu") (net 27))
 (segment (start 147.182 61.447) (end 147.182 78.0618) (width 0.5) (layer "B.Cu") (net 35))
 (segment (start 147.182 78.0618) (end 155.31 86.19) (width 0.5) (layer "B.Cu") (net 35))
 (segment (start 146.605 60.87) (end 147.182 61.447) (width 0.5) (layer "B.Cu") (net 35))
 (segment (start 160.5 79.5) (end 156.765 75.765) (width 0.5) (layer "B.Cu") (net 38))
 (segment (start 160.775454 81.775454) (end 160.5 81.5) (width 0.5) (layer "B.Cu") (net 38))
 (segment (start 165 85.47894) (end 164.999998 85.47894) (width 0.5) (layer "B.Cu") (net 38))
 (segment (start 160.5 81.5) (end 160.5 79.5) (width 0.5) (layer "B.Cu") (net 38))
 (segment (start 164 85) (end 160.775454 81.775454) (width 0.5) (layer "B.Cu") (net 38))
 (segment (start 156.765 75.765) (end 156.765 60.87) (width 0.5) (layer "B.Cu") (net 38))
 (segment (start 164.999998 85.47894) (end 164.521058 85) (width 0.5) (layer "B.Cu") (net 38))
 (segment (start 165 85.46) (end 165 85.47894) (width 0.5) (layer "B.Cu") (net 38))
 (segment (start 164.521058 85) (end 164 85) (width 0.5) (layer "B.Cu") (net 38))
 (segment (start 136.76 78.7077) (end 134.772 76.7195) (width 0.5) (layer "F.Cu") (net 1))
 (segment (start 127.052 69) (end 126.54 69) (width 0.5) (layer "F.Cu") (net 1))
 (segment (start 136.79102 78.73872) (end 136.76 78.7077) (width 0.5) (layer "F.Cu") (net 1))
 (segment (start 120.718 78.5607) (end 125.4393 78.5607) (width 0.5) (layer "F.Cu") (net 1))
 (segment (start 125.4393 78.5607) (end 131.026 72.974) (width 0.5) (layer "F.Cu") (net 1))
 (segment (start 114 85.2791) (end 120.718 78.5607) (width 0.5) (layer "F.Cu") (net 1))
 (segment (start 152.93892 78.73892) (end 152.93892 78.73872) (width 0.5) (layer "F.Cu") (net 1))
 (segment (start 114 86) (end 114 85.2791) (width 0.5) (layer "F.Cu") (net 1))
 (segment (start 130.335 72.283) (end 127.052 69) (width 0.5) (layer "F.Cu") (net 1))
 (segment (start 131.026 72.974) (end 130.335 72.283) (width 0.5) (layer "F.Cu") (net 1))
 (segment (start 155.31 81.11) (end 152.93892 78.73892) (width 0.5) (layer "F.Cu") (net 1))
 (segment (start 152.93892 78.73872) (end 136.79102 78.73872) (width 0.5) (layer "F.Cu") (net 1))
 (segment (start 134.772 76.7195) (end 130.335 72.283) (width 0.5) (layer "F.Cu") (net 1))
 (segment (start 131.0491 101.1941) (end 121.5096 101.1941) (width 0.5) (layer "B.Cu") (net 1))
 (segment (start 112 88) (end 114 86) (width 0.5) (layer "B.Cu") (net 1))
 (segment (start 121.5096 101.1941) (end 112 91.6845) (width 0.5) (layer "B.Cu") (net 1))
 (segment (start 138.985 109.13) (end 131.0491 101.1941) (width 0.5) (layer "B.Cu") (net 1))
 (segment (start 112 91.6845) (end 112 88) (width 0.5) (layer "B.Cu") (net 1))
 (segment (start 132.13 60.87) (end 132.385 60.87) (width 0.5) (layer "B.Cu") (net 24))
 (segment (start 124 69) (end 132.13 60.87) (width 0.5) (layer "B.Cu") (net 24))
 (segment (start 150.293 109.13) (end 148.163 107) (width 0.5) (layer "F.Cu") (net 3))
 (segment (start 151.685 109.13) (end 150.293 109.13) (width 0.5) (layer "F.Cu") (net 3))
 (segment (start 124 107) (end 114 97) (width 0.5) (layer "F.Cu") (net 3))
 (segment (start 148.163 107) (end 124 107) (width 0.5) (layer "F.Cu") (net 3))
 (segment (start 114 97) (end 114 91.08) (width 0.5) (layer "F.Cu") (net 3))
 (segment (start 163 62.025) (end 161.845 60.87) (width 0.5) (layer "B.Cu") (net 37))
 (segment (start 164.42 82.92) (end 163 81.5) (width 0.5) (layer "B.Cu") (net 37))
 (segment (start 163 81.5) (end 163 62.025) (width 0.5) (layer "B.Cu") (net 37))
 (segment (start 165 82.92) (end 164.42 82.92) (width 0.5) (layer "B.Cu") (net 37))
 (segment (start 159.305 98.775) (end 165 93.08) (width 0.5) (layer "B.Cu") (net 41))
 (segment (start 159.305 109.13) (end 159.305 98.775) (width 0.5) (layer "B.Cu") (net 41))
 (segment (start 152.202 61.387) (end 151.685 60.87) (width 0.5) (layer "B.Cu") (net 33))
 (segment (start 152.202 73.702) (end 152.202 61.387) (width 0.5) (layer "B.Cu") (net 33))
 (segment (start 153.384 74.884) (end 152.202 73.702) (width 0.5) (layer "B.Cu") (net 33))
 (segment (start 158.5 90.62) (end 158.5 80.189354) (width 0.5) (layer "B.Cu") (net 33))
 (segment (start 155.31 93.81) (end 158.5 90.62) (width 0.5) (layer "B.Cu") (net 33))
 (segment (start 158.5 80.189354) (end 153.384 75.073354) (width 0.5) (layer "B.Cu") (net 33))
 (segment (start 153.384 75.073354) (end 153.384 74.884) (width 0.5) (layer "B.Cu") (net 33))
 (segment (start 165 61.485) (end 164.385 60.87) (width 0.5) (layer "B.Cu") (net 36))
 (segment (start 165 80.38) (end 165 61.485) (width 0.5) (layer "B.Cu") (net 36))
 (segment (start 137.465 60.87) (end 137.465 63.2834) (width 0.5) (layer "B.Cu") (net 4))
 (segment (start 137.465 63.2834) (end 131.69 69.0584) (width 0.5) (layer "B.Cu") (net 4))
 (segment (start 131.69 69.0584) (end 131.69 69.5) (width 0.5) (layer "B.Cu") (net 4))
 (segment (start 139.31 69.5) (end 146.89 77.08) (width 0.5) (layer "F.Cu") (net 5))
 (segment (start 146.89 77.08) (end 160.5 77.08) (width 0.5) (layer "F.Cu") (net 5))
 (segment (start 146.54 74.54) (end 145.5 73.5) (width 0.5) (layer "F.Cu") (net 23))
 (segment (start 160.5 74.54) (end 146.54 74.54) (width 0.5) (layer "F.Cu") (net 23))
 (segment (start 150.85 69.46) (end 150.81 69.5) (width 0.5) (layer "F.Cu") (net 26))
 (segment (start 160.5 69.46) (end 150.85 69.46) (width 0.5) (layer "F.Cu") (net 26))
 (segment (start 144.12 96.2) (end 147.54 96.2) (width 0.5) (layer "F.Cu") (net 15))
 (segment (start 147.54 96.2) (end 147.69 96.35) (width 0.5) (layer "F.Cu") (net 15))
 (segment (start 147.69 86.19) (end 144.27 86.19) (width 0.5) (layer "F.Cu") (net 19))
 (segment (start 144.27 86.19) (end 144.12 86.04) (width 0.5) (layer "F.Cu") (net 19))
 (segment (start 144.27 83.65) (end 144.12 83.5) (width 0.5) (layer "F.Cu") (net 20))
 (segment (start 147.69 83.65) (end 144.27 83.65) (width 0.5) (layer "F.Cu") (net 20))
 (segment (start 147.69 93.81) (end 144.27 93.81) (width 0.5) (layer "F.Cu") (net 16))
 (segment (start 144.27 93.81) (end 144.12 93.66) (width 0.5) (layer "F.Cu") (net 16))
 (segment (start 144.12 91.12) (end 147.54 91.12) (width 0.5) (layer "F.Cu") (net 17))
 (segment (start 147.54 91.12) (end 147.69 91.27) (width 0.5) (layer "F.Cu") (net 17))
 (segment (start 147.54 88.58) (end 147.69 88.73) (width 0.5) (layer "F.Cu") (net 18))
 (segment (start 144.12 88.58) (end 147.54 88.58) (width 0.5) (layer "F.Cu") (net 18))
 (segment (start 147.54 80.96) (end 147.69 81.11) (width 0.5) (layer "B.Cu") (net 21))
 (segment (start 144.12 80.96) (end 147.54 80.96) (width 0.5) (layer "B.Cu") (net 21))
 (segment (start 148.5 101) (end 146.38 101) (width 0.5) (layer "F.Cu") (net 14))
 (segment (start 149.93 89.03) (end 149.93 99.57) (width 0.5) (layer "F.Cu") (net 14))
 (segment (start 146.38 101) (end 144.12 98.74) (width 0.5) (layer "F.Cu") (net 14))
 (segment (start 155.31 83.65) (end 149.93 89.03) (width 0.5) (layer "F.Cu") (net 14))
 (segment (start 149.93 99.57) (end 148.5 101) (width 0.5) (layer "F.Cu") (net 14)))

